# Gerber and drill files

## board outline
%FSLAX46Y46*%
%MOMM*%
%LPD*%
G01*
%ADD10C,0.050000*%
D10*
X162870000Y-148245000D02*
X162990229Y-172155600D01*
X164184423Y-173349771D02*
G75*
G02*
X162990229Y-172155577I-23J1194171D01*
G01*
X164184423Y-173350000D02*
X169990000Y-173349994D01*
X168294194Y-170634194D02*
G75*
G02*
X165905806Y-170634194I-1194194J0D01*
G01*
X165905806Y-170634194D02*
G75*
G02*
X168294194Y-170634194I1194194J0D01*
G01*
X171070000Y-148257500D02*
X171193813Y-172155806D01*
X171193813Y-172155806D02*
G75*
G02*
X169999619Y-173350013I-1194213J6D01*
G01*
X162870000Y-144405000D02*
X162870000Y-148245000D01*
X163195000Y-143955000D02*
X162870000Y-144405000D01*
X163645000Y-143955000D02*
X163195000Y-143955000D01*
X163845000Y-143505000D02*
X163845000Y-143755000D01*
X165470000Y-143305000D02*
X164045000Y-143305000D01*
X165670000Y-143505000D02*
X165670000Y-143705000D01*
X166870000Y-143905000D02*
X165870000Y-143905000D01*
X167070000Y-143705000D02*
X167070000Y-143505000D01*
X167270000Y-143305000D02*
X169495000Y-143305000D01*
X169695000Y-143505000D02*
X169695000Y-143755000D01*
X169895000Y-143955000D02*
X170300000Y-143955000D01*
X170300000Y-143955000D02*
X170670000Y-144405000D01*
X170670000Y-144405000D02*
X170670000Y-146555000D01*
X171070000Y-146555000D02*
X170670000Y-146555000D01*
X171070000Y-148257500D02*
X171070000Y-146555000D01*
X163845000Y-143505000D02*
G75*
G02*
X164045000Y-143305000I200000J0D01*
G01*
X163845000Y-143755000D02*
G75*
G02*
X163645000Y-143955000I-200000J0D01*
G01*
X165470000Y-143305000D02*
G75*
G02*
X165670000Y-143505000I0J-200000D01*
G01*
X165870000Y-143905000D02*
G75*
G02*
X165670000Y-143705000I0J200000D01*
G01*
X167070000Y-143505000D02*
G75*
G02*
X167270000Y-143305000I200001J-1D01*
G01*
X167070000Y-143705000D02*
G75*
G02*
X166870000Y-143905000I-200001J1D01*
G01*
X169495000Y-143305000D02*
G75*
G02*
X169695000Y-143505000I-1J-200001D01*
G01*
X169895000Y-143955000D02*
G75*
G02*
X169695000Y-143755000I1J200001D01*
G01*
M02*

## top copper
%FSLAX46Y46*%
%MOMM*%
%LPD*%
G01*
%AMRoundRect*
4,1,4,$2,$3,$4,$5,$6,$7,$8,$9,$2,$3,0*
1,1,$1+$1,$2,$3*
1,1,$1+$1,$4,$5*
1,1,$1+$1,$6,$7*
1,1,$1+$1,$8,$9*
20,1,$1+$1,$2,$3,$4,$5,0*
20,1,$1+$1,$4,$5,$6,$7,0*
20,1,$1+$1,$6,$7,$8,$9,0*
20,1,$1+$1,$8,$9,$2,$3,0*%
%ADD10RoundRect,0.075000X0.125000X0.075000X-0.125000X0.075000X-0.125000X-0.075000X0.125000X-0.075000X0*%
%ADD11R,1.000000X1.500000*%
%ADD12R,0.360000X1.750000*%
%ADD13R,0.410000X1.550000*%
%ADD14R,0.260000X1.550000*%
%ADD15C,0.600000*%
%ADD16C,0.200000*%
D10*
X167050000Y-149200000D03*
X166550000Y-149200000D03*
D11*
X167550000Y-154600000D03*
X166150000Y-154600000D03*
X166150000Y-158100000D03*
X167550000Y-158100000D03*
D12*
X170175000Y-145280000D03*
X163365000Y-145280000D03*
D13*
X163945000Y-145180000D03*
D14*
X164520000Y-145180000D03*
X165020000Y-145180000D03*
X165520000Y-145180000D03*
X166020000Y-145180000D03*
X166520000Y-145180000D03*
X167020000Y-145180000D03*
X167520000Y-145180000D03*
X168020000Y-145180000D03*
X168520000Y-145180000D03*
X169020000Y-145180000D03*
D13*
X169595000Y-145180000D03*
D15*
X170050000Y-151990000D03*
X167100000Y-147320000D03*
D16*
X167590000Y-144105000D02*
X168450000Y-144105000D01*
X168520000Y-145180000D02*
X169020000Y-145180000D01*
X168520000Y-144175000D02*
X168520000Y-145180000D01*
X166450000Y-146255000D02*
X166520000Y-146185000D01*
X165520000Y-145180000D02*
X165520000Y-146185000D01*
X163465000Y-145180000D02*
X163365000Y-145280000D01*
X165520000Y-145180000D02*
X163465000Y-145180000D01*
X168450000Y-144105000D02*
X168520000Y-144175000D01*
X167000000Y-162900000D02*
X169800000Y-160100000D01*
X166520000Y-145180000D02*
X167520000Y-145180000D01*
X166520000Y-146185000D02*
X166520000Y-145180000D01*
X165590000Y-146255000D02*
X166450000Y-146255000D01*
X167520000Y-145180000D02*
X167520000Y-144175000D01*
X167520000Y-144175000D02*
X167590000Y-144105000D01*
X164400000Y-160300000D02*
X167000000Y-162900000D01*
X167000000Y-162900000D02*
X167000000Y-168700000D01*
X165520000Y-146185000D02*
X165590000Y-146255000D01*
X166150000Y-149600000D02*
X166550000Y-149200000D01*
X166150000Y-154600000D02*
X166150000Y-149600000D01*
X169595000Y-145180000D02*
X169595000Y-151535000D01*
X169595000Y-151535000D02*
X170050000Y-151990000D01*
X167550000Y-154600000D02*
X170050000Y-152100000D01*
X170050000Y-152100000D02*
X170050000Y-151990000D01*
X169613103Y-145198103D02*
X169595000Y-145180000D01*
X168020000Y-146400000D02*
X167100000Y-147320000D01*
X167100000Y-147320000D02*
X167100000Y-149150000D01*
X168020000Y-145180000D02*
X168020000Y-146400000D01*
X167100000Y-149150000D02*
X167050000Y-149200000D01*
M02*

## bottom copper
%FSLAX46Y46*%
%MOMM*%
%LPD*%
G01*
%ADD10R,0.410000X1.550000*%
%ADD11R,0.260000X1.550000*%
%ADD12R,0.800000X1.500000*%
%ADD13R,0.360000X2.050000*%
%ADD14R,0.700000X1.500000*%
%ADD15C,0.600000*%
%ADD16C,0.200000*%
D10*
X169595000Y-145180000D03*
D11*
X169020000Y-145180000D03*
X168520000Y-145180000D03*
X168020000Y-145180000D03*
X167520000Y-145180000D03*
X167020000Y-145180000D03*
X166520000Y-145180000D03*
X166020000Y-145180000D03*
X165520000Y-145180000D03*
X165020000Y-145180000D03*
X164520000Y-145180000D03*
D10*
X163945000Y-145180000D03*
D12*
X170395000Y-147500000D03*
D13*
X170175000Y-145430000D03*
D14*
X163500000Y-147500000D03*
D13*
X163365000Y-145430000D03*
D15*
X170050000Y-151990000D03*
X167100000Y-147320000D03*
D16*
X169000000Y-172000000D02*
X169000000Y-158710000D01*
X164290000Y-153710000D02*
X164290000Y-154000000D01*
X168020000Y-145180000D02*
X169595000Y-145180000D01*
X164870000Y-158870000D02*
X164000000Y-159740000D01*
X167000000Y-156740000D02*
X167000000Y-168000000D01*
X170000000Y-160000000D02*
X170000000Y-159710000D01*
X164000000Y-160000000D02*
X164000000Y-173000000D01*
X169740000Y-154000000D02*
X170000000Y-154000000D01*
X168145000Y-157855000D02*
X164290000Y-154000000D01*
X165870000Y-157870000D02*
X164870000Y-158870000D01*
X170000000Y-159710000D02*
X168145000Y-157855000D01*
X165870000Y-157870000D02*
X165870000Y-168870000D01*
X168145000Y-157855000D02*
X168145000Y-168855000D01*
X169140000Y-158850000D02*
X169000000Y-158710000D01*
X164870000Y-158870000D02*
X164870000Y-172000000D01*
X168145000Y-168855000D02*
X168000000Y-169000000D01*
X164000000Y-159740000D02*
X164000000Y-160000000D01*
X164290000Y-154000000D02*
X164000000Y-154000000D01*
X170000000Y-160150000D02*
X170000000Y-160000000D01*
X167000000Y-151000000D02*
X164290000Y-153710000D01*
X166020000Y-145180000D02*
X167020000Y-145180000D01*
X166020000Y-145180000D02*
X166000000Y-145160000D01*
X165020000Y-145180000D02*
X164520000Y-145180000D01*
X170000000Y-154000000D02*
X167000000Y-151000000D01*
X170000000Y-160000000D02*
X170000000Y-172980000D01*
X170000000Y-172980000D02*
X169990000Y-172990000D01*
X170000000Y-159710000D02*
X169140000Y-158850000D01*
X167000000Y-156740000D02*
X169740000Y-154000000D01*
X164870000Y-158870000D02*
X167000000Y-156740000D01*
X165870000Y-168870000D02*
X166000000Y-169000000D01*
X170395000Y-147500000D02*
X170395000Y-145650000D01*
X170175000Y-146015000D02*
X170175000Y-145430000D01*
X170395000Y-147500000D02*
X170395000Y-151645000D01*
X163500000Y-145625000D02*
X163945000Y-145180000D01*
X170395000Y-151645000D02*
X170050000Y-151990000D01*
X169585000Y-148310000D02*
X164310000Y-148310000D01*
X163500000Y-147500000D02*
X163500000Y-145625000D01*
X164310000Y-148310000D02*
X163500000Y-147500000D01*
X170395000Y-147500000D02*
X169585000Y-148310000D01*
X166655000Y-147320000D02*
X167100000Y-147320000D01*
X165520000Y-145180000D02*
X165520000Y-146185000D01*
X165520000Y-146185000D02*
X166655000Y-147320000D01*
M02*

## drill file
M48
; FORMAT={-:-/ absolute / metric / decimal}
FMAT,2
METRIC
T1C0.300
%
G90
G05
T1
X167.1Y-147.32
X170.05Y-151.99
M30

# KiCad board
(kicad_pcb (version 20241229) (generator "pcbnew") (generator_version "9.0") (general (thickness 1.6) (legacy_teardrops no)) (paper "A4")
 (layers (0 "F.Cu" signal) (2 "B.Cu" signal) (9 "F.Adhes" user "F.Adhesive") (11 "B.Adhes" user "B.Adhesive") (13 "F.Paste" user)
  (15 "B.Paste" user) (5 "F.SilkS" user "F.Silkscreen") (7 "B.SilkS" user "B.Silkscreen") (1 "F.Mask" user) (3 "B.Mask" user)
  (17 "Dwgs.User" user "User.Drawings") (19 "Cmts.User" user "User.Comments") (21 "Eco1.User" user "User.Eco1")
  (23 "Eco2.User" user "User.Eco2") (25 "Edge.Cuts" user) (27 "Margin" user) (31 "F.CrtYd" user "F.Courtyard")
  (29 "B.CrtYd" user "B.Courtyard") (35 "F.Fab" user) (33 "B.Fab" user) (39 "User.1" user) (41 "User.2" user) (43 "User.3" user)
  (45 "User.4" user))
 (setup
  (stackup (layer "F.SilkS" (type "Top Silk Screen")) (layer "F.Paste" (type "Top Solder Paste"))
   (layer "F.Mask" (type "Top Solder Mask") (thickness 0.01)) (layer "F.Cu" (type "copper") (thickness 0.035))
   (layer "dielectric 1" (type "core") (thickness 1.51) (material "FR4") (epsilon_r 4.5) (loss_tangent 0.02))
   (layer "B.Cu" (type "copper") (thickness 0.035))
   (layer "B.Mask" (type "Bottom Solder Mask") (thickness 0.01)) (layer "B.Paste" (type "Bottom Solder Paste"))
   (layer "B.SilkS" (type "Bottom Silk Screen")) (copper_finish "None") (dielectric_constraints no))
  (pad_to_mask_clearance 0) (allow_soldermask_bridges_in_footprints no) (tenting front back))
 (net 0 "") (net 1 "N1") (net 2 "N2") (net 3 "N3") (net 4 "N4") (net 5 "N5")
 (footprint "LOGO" (layer "F.Cu") (at 167 156)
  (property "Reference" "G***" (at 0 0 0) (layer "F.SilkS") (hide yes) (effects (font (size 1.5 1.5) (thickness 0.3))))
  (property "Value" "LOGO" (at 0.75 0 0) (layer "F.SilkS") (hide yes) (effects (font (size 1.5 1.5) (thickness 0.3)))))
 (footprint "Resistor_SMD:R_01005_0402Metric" (layer "F.Cu") (at 166.8 149.2 180)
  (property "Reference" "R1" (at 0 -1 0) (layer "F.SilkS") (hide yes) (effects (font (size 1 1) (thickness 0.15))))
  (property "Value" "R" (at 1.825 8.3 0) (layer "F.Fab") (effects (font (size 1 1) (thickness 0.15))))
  (pad "" smd roundrect (at -0.275 0 180) (size 0.27 0.27) (layers "F.Paste") (roundrect_rratio 0.25))
  (pad "" smd roundrect (at 0.275 0 180) (size 0.27 0.27) (layers "F.Paste") (roundrect_rratio 0.25))
  (pad "1" smd roundrect (at -0.25 0 180) (size 0.4 0.3) (layers "F.Cu" "F.Mask") (roundrect_rratio 0.25) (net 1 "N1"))
  (pad "2" smd roundrect (at 0.25 0 180) (size 0.4 0.3) (layers "F.Cu" "F.Mask") (roundrect_rratio 0.25) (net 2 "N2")))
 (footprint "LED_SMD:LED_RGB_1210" (layer "F.Cu") (at 166.85 156.35 -90)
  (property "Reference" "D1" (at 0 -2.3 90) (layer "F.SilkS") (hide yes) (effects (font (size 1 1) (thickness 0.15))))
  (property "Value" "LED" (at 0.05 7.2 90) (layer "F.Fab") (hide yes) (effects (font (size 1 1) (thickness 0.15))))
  (pad "1" smd rect (at -1.75 -0.7 90) (size 1.5 1) (layers "F.Cu" "F.Mask" "F.Paste") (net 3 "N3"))
  (pad "2" smd rect (at -1.75 0.7 90) (size 1.5 1) (layers "F.Cu" "F.Mask" "F.Paste") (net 2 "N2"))
  (pad "3" smd rect (at 1.75 0.7 90) (size 1.5 1) (layers "F.Cu" "F.Mask" "F.Paste"))
  (pad "4" smd rect (at 1.75 -0.7 90) (size 1.5 1) (layers "F.Cu" "F.Mask" "F.Paste")))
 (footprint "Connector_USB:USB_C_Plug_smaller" (layer "F.Cu") (at 166.77 146.3275 180)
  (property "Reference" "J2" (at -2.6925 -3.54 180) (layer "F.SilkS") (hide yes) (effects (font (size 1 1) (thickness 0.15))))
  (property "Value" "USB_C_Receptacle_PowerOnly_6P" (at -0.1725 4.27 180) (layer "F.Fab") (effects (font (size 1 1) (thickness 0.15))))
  (fp_line (start 3.9 1.9225) (end 3.9 -1.9175) (stroke (width 0.05) (type solid)) (layer "Edge.Cuts"))
  (fp_line (start 3.575 2.3725) (end 3.9 1.9225) (stroke (width 0.05) (type solid)) (layer "Edge.Cuts"))
  (fp_line (start 3.125 2.3725) (end 3.575 2.3725) (stroke (width 0.05) (type solid)) (layer "Edge.Cuts"))
  (fp_line (start 2.925 2.8225) (end 2.925 2.5725) (stroke (width 0.05) (type solid)) (layer "Edge.Cuts"))
  (fp_line (start 1.3 3.0225) (end 2.725 3.0225) (stroke (width 0.05) (type solid)) (layer "Edge.Cuts"))
  (fp_line (start 1.1 2.8225) (end 1.1 2.6225) (stroke (width 0.05) (type solid)) (layer "Edge.Cuts"))
  (fp_line (start -0.1 2.4225) (end 0.9 2.4225) (stroke (width 0.05) (type solid)) (layer "Edge.Cuts"))
  (fp_line (start -0.3 2.6225) (end -0.3 2.8225) (stroke (width 0.05) (type solid)) (layer "Edge.Cuts"))
  (fp_line (start -0.5 3.0225) (end -2.725 3.0225) (stroke (width 0.05) (type solid)) (layer "Edge.Cuts"))
  (fp_line (start -2.925 2.8225) (end -2.925 2.5725) (stroke (width 0.05) (type solid)) (layer "Edge.Cuts"))
  (fp_line (start -3.125 2.3725) (end -3.53 2.3725) (stroke (width 0.05) (type solid)) (layer "Edge.Cuts"))
  (fp_line (start -3.53 2.3725) (end -3.9 1.9225) (stroke (width 0.05) (type solid)) (layer "Edge.Cuts"))
  (fp_line (start -3.9 1.9225) (end -3.9 -0.2275) (stroke (width 0.05) (type solid)) (layer "Edge.Cuts"))
  (fp_line (start -4.3 -0.2275) (end -3.9 -0.2275) (stroke (width 0.05) (type solid)) (layer "Edge.Cuts"))
  (fp_line (start -4.3 -1.93) (end -4.3 -0.2275) (stroke (width 0.05) (type solid)) (layer "Edge.Cuts"))
  (fp_arc (start 2.925 2.8225) (mid 2.866421 2.963921) (end 2.725 3.0225) (stroke (width 0.05) (type solid)) (layer "Edge.Cuts"))
  (fp_arc (start 2.925 2.5725) (mid 2.983579 2.431079) (end 3.125 2.3725) (stroke (width 0.05) (type solid)) (layer "Edge.Cuts"))
  (fp_arc (start 1.3 3.0225) (mid 1.158579 2.963921) (end 1.1 2.8225) (stroke (width 0.05) (type solid)) (layer "Edge.Cuts"))
  (fp_arc (start 0.9 2.4225) (mid 1.041421 2.481079) (end 1.1 2.6225) (stroke (width 0.05) (type solid)) (layer "Edge.Cuts"))
  (fp_arc (start -0.3 2.8225) (mid -0.358579 2.963921) (end -0.5 3.0225) (stroke (width 0.05) (type solid)) (layer "Edge.Cuts"))
  (fp_arc (start -0.3 2.6225) (mid -0.241421 2.481079) (end -0.1 2.4225) (stroke (width 0.05) (type solid)) (layer "Edge.Cuts"))
  (fp_arc (start -2.725 3.0225) (mid -2.866421 2.963921) (end -2.925 2.8225) (stroke (width 0.05) (type solid)) (layer "Edge.Cuts"))
  (fp_arc (start -3.125 2.3725) (mid -2.983579 2.431079) (end -2.925 2.5725) (stroke (width 0.05) (type solid)) (layer "Edge.Cuts"))
  (pad "" smd rect (at -3.405 1.0475 180) (size 0.36 1.75) (layers "F.Cu" "F.Mask"))
  (pad "" smd rect (at 3.405 1.0475 180) (size 0.36 1.75) (layers "F.Cu" "F.Mask"))
  (pad "A1" smd rect (at 2.825 1.1475 180) (size 0.41 1.55) (layers "F.Cu" "F.Mask" "F.Paste"))
  (pad "A2" smd rect (at 2.25 1.1475 180) (size 0.26 1.55) (layers "F.Cu" "F.Mask" "F.Paste"))
  (pad "A3" smd rect (at 1.75 1.1475 180) (size 0.26 1.55) (layers "F.Cu" "F.Mask" "F.Paste"))
  (pad "A4" smd rect (at 1.25 1.1475 180) (size 0.26 1.55) (layers "F.Cu" "F.Mask" "F.Paste"))
  (pad "A5" smd rect (at 0.75 1.1475 180) (size 0.26 1.55) (layers "F.Cu" "F.Mask" "F.Paste") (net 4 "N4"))
  (pad "A6" smd rect (at 0.25 1.1475) (size 0.26 1.55) (layers "F.Cu" "F.Mask" "F.Paste"))
  (pad "A7" smd rect (at -0.25 1.1475) (size 0.26 1.55) (layers "F.Cu" "F.Mask" "F.Paste"))
  (pad "A8" smd rect (at -0.75 1.1475 180) (size 0.26 1.55) (layers "F.Cu" "F.Mask" "F.Paste"))
  (pad "A9" smd rect (at -1.25 1.1475 180) (size 0.26 1.55) (layers "F.Cu" "F.Mask" "F.Paste") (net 1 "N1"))
  (pad "A10" smd rect (at -1.75 1.1475 180) (size 0.26 1.55) (layers "F.Cu" "F.Mask" "F.Paste"))
  (pad "A11" smd rect (at -2.25 1.1475 180) (size 0.26 1.55) (layers "F.Cu" "F.Mask" "F.Paste"))
  (pad "A12" smd rect (at -2.825 1.1475 180) (size 0.41 1.55) (layers "F.Cu" "F.Mask" "F.Paste") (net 3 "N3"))
  (pad "B1" smd rect (at -2.825 1.1475 180) (size 0.41 1.55) (layers "B.Cu" "B.Mask" "B.Paste"))
  (pad "B2" smd rect (at -2.25 1.1475 180) (size 0.26 1.55) (layers "B.Cu" "B.Mask" "B.Paste"))
  (pad "B3" smd rect (at -1.75 1.1475 180) (size 0.26 1.55) (layers "B.Cu" "B.Mask" "B.Paste"))
  (pad "B4" smd rect (at -1.25 1.1475 180) (size 0.26 1.55) (layers "B.Cu" "B.Mask" "B.Paste"))
  (pad "B5" smd rect (at -0.75 1.1475 180) (size 0.26 1.55) (layers "B.Cu" "B.Mask" "B.Paste") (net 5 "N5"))
  (pad "B6" smd rect (at -0.25 1.1475) (size 0.26 1.55) (layers "B.Cu" "B.Mask" "B.Paste"))
  (pad "B7" smd rect (at 0.25 1.1475 180) (size 0.26 1.55) (layers "B.Cu" "B.Mask" "B.Paste"))
  (pad "B8" smd rect (at 0.75 1.1475 180) (size 0.26 1.55) (layers "B.Cu" "B.Mask" "B.Paste"))
  (pad "B9" smd rect (at 1.25 1.1475 180) (size 0.26 1.55) (layers "B.Cu" "B.Mask" "B.Paste") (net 1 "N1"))
  (pad "B10" smd rect (at 1.75 1.1475 180) (size 0.26 1.55) (layers "B.Cu" "B.Mask" "B.Paste"))
  (pad "B11" smd rect (at 2.25 1.1475 180) (size 0.26 1.55) (layers "B.Cu" "B.Mask" "B.Paste"))
  (pad "B12" smd rect (at 2.825 1.1475 180) (size 0.41 1.55) (layers "B.Cu" "B.Mask" "B.Paste") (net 3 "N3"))
  (pad "S1" smd rect (at -3.625 -1.1725 180) (size 0.8 1.5) (layers "B.Cu" "B.Mask" "B.Paste") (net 3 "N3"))
  (pad "S1" smd rect (at -3.405 0.8975 180) (size 0.36 2.05) (layers "B.Cu" "B.Mask" "B.Paste") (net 3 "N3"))
  (pad "S1" smd rect (at 3.27 -1.1725) (size 0.7 1.5) (layers "B.Cu" "B.Mask" "B.Paste") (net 3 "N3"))
  (pad "S1" smd rect (at 3.405 0.8975 180) (size 0.36 2.05) (layers "B.Cu" "B.Mask" "B.Paste") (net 3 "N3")))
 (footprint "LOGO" (layer "B.Cu") (at 167 156 180)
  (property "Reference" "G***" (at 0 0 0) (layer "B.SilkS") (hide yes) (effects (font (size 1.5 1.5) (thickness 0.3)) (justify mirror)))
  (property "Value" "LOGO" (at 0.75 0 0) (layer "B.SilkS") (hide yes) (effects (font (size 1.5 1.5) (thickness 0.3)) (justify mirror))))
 (gr_line (start 162.87 148.245) (end 162.990229 172.1556) (stroke (width 0.05) (type default)) (layer "Edge.Cuts"))
 (gr_arc (start 164.184423 173.349771) (mid 163.34 173) (end 162.990229 172.155577) (stroke (width 0.05) (type default)) (layer "Edge.Cuts"))
 (gr_line (start 164.184423 173.35) (end 169.99 173.349994) (stroke (width 0.05) (type default)) (layer "Edge.Cuts"))
 (gr_circle (center 167.1 170.634194) (end 167.2 169.444194) (stroke (width 0.05) (type default)) (fill no) (layer "Edge.Cuts"))
 (gr_line (start 171.07 148.2575) (end 171.193813 172.155806) (stroke (width 0.05) (type default)) (layer "Edge.Cuts"))
 (gr_arc (start 171.193813 172.155806) (mid 170.844042 173.000229) (end 169.999619 173.35) (stroke (width 0.05) (type default))
  (layer "Edge.Cuts"))
 (segment (start 167.59 144.105) (end 168.45 144.105) (width 0.2) (layer "F.Cu") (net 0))
 (segment (start 168.52 145.18) (end 169.02 145.18) (width 0.2) (layer "F.Cu") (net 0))
 (segment (start 168.52 144.175) (end 168.52 145.18) (width 0.2) (layer "F.Cu") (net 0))
 (segment (start 166.45 146.255) (end 166.52 146.185) (width 0.2) (layer "F.Cu") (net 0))
 (segment (start 165.52 145.18) (end 165.52 146.185) (width 0.2) (layer "F.Cu") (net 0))
 (segment (start 163.465 145.18) (end 163.365 145.28) (width 0.2) (layer "F.Cu") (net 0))
 (segment (start 165.52 145.18) (end 163.465 145.18) (width 0.2) (layer "F.Cu") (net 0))
 (segment (start 168.45 144.105) (end 168.52 144.175) (width 0.2) (layer "F.Cu") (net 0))
 (segment (start 167 162.9) (end 169.8 160.1) (width 0.2) (layer "F.Cu") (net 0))
 (segment (start 166.52 145.18) (end 167.52 145.18) (width 0.2) (layer "F.Cu") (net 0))
 (segment (start 166.52 146.185) (end 166.52 145.18) (width 0.2) (layer "F.Cu") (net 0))
 (segment (start 165.59 146.255) (end 166.45 146.255) (width 0.2) (layer "F.Cu") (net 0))
 (segment (start 167.52 145.18) (end 167.52 144.175) (width 0.2) (layer "F.Cu") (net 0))
 (segment (start 167.52 144.175) (end 167.59 144.105) (width 0.2) (layer "F.Cu") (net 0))
 (segment (start 164.4 160.3) (end 167 162.9) (width 0.2) (layer "F.Cu") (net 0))
 (segment (start 167 162.9) (end 167 168.7) (width 0.2) (layer "F.Cu") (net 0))
 (segment (start 165.52 146.185) (end 165.59 146.255) (width 0.2) (layer "F.Cu") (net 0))
 (segment (start 169 172) (end 169 158.71) (width 0.2) (layer "B.Cu") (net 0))
 (segment (start 164.29 153.71) (end 164.29 154) (width 0.2) (layer "B.Cu") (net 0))
 (segment (start 168.02 145.18) (end 169.595 145.18) (width 0.2) (layer "B.Cu") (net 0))
 (segment (start 164.87 158.87) (end 164 159.74) (width 0.2) (layer "B.Cu") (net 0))
 (segment (start 167 156.74) (end 167 168) (width 0.2) (layer "B.Cu") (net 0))
 (segment (start 170 160) (end 170 159.71) (width 0.2) (layer "B.Cu") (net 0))
 (segment (start 164 160) (end 164 173) (width 0.2) (layer "B.Cu") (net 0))
 (segment (start 169.74 154) (end 170 154) (width 0.2) (layer "B.Cu") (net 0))
 (segment (start 168.145 157.855) (end 164.29 154) (width 0.2) (layer "B.Cu") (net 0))
 (segment (start 165.87 157.87) (end 164.87 158.87) (width 0.2) (layer "B.Cu") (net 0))
 (segment (start 170 159.71) (end 168.145 157.855) (width 0.2) (layer "B.Cu") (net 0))
 (segment (start 165.87 157.87) (end 165.87 168.87) (width 0.2) (layer "B.Cu") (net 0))
 (segment (start 168.145 157.855) (end 168.145 168.855) (width 0.2) (layer "B.Cu") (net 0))
 (segment (start 169.14 158.85) (end 169 158.71) (width 0.2) (layer "B.Cu") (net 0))
 (segment (start 164.87 158.87) (end 164.87 172) (width 0.2) (layer "B.Cu") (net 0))
 (segment (start 168.145 168.855) (end 168 169) (width 0.2) (layer "B.Cu") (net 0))
 (segment (start 164 159.74) (end 164 160) (width 0.2) (layer "B.Cu") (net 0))
 (segment (start 164.29 154) (end 164 154) (width 0.2) (layer "B.Cu") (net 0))
 (segment (start 170 160.15) (end 170 160) (width 0.2) (layer "B.Cu") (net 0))
 (segment (start 167 151) (end 164.29 153.71) (width 0.2) (layer "B.Cu") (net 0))
 (segment (start 166.02 145.18) (end 167.02 145.18) (width 0.2) (layer "B.Cu") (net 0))
 (segment (start 166.02 145.18) (end 166 145.16) (width 0.2) (layer "B.Cu") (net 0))
 (segment (start 165.02 145.18) (end 164.52 145.18) (width 0.2) (layer "B.Cu") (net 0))
 (segment (start 170 154) (end 167 151) (width 0.2) (layer "B.Cu") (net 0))
 (segment (start 170 160) (end 170 172.98) (width 0.2) (layer "B.Cu") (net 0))
 (segment (start 170 172.98) (end 169.99 172.99) (width 0.2) (layer "B.Cu") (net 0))
 (segment (start 170 159.71) (end 169.14 158.85) (width 0.2) (layer "B.Cu") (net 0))
 (segment (start 167 156.74) (end 169.74 154) (width 0.2) (layer "B.Cu") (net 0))
 (segment (start 164.87 158.87) (end 167 156.74) (width 0.2) (layer "B.Cu") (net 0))
 (segment (start 165.87 168.87) (end 166 169) (width 0.2) (layer "B.Cu") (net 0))
 (segment (start 166.15 149.6) (end 166.55 149.2) (width 0.2) (layer "F.Cu") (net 2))
 (segment (start 166.15 154.6) (end 166.15 149.6) (width 0.2) (layer "F.Cu") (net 2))
 (segment (start 169.595 145.18) (end 169.595 151.535) (width 0.2) (layer "F.Cu") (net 3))
 (segment (start 169.595 151.535) (end 170.05 151.99) (width 0.2) (layer "F.Cu") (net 3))
 (segment (start 167.55 154.6) (end 170.05 152.1) (width 0.2) (layer "F.Cu") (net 3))
 (segment (start 170.05 152.1) (end 170.05 151.99) (width 0.2) (layer "F.Cu") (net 3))
 (segment (start 169.613103 145.198103) (end 169.595 145.18) (width 0.2) (layer "F.Cu") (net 3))
 (via (at 170.05 151.99) (size 0.6) (drill 0.3) (layers "F.Cu" "B.Cu") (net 3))
 (segment (start 170.395 147.5) (end 170.395 145.65) (width 0.2) (layer "B.Cu") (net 3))
 (segment (start 170.175 146.015) (end 170.175 145.43) (width 0.2) (layer "B.Cu") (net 3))
 (segment (start 170.395 147.5) (end 170.395 151.645) (width 0.2) (layer "B.Cu") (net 3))
 (segment (start 163.5 145.625) (end 163.945 145.18) (width 0.2) (layer "B.Cu") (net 3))
 (segment (start 170.395 151.645) (end 170.05 151.99) (width 0.2) (layer "B.Cu") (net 3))
 (segment (start 169.585 148.31) (end 164.31 148.31) (width 0.2) (layer "B.Cu") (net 3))
 (segment (start 163.5 147.5) (end 163.5 145.625) (width 0.2) (layer "B.Cu") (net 3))
 (segment (start 164.31 148.31) (end 163.5 147.5) (width 0.2) (layer "B.Cu") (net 3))
 (segment (start 170.395 147.5) (end 169.585 148.31) (width 0.2) (layer "B.Cu") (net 3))
 (segment (start 168.02 146.4) (end 167.1 147.32) (width 0.2) (layer "F.Cu") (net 1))
 (segment (start 167.1 147.32) (end 167.1 149.15) (width 0.2) (layer "F.Cu") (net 1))
 (segment (start 168.02 145.18) (end 168.02 146.4) (width 0.2) (layer "F.Cu") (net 1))
 (segment (start 167.1 149.15) (end 167.05 149.2) (width 0.2) (layer "F.Cu") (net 1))
 (via (at 167.1 147.32) (size 0.6) (drill 0.3) (layers "F.Cu" "B.Cu") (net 1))
 (segment (start 166.655 147.32) (end 167.1 147.32) (width 0.2) (layer "B.Cu") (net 1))
 (segment (start 165.52 145.18) (end 165.52 146.185) (width 0.2) (layer "B.Cu") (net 1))
 (segment (start 165.52 146.185) (end 166.655 147.32) (width 0.2) (layer "B.Cu") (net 1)))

